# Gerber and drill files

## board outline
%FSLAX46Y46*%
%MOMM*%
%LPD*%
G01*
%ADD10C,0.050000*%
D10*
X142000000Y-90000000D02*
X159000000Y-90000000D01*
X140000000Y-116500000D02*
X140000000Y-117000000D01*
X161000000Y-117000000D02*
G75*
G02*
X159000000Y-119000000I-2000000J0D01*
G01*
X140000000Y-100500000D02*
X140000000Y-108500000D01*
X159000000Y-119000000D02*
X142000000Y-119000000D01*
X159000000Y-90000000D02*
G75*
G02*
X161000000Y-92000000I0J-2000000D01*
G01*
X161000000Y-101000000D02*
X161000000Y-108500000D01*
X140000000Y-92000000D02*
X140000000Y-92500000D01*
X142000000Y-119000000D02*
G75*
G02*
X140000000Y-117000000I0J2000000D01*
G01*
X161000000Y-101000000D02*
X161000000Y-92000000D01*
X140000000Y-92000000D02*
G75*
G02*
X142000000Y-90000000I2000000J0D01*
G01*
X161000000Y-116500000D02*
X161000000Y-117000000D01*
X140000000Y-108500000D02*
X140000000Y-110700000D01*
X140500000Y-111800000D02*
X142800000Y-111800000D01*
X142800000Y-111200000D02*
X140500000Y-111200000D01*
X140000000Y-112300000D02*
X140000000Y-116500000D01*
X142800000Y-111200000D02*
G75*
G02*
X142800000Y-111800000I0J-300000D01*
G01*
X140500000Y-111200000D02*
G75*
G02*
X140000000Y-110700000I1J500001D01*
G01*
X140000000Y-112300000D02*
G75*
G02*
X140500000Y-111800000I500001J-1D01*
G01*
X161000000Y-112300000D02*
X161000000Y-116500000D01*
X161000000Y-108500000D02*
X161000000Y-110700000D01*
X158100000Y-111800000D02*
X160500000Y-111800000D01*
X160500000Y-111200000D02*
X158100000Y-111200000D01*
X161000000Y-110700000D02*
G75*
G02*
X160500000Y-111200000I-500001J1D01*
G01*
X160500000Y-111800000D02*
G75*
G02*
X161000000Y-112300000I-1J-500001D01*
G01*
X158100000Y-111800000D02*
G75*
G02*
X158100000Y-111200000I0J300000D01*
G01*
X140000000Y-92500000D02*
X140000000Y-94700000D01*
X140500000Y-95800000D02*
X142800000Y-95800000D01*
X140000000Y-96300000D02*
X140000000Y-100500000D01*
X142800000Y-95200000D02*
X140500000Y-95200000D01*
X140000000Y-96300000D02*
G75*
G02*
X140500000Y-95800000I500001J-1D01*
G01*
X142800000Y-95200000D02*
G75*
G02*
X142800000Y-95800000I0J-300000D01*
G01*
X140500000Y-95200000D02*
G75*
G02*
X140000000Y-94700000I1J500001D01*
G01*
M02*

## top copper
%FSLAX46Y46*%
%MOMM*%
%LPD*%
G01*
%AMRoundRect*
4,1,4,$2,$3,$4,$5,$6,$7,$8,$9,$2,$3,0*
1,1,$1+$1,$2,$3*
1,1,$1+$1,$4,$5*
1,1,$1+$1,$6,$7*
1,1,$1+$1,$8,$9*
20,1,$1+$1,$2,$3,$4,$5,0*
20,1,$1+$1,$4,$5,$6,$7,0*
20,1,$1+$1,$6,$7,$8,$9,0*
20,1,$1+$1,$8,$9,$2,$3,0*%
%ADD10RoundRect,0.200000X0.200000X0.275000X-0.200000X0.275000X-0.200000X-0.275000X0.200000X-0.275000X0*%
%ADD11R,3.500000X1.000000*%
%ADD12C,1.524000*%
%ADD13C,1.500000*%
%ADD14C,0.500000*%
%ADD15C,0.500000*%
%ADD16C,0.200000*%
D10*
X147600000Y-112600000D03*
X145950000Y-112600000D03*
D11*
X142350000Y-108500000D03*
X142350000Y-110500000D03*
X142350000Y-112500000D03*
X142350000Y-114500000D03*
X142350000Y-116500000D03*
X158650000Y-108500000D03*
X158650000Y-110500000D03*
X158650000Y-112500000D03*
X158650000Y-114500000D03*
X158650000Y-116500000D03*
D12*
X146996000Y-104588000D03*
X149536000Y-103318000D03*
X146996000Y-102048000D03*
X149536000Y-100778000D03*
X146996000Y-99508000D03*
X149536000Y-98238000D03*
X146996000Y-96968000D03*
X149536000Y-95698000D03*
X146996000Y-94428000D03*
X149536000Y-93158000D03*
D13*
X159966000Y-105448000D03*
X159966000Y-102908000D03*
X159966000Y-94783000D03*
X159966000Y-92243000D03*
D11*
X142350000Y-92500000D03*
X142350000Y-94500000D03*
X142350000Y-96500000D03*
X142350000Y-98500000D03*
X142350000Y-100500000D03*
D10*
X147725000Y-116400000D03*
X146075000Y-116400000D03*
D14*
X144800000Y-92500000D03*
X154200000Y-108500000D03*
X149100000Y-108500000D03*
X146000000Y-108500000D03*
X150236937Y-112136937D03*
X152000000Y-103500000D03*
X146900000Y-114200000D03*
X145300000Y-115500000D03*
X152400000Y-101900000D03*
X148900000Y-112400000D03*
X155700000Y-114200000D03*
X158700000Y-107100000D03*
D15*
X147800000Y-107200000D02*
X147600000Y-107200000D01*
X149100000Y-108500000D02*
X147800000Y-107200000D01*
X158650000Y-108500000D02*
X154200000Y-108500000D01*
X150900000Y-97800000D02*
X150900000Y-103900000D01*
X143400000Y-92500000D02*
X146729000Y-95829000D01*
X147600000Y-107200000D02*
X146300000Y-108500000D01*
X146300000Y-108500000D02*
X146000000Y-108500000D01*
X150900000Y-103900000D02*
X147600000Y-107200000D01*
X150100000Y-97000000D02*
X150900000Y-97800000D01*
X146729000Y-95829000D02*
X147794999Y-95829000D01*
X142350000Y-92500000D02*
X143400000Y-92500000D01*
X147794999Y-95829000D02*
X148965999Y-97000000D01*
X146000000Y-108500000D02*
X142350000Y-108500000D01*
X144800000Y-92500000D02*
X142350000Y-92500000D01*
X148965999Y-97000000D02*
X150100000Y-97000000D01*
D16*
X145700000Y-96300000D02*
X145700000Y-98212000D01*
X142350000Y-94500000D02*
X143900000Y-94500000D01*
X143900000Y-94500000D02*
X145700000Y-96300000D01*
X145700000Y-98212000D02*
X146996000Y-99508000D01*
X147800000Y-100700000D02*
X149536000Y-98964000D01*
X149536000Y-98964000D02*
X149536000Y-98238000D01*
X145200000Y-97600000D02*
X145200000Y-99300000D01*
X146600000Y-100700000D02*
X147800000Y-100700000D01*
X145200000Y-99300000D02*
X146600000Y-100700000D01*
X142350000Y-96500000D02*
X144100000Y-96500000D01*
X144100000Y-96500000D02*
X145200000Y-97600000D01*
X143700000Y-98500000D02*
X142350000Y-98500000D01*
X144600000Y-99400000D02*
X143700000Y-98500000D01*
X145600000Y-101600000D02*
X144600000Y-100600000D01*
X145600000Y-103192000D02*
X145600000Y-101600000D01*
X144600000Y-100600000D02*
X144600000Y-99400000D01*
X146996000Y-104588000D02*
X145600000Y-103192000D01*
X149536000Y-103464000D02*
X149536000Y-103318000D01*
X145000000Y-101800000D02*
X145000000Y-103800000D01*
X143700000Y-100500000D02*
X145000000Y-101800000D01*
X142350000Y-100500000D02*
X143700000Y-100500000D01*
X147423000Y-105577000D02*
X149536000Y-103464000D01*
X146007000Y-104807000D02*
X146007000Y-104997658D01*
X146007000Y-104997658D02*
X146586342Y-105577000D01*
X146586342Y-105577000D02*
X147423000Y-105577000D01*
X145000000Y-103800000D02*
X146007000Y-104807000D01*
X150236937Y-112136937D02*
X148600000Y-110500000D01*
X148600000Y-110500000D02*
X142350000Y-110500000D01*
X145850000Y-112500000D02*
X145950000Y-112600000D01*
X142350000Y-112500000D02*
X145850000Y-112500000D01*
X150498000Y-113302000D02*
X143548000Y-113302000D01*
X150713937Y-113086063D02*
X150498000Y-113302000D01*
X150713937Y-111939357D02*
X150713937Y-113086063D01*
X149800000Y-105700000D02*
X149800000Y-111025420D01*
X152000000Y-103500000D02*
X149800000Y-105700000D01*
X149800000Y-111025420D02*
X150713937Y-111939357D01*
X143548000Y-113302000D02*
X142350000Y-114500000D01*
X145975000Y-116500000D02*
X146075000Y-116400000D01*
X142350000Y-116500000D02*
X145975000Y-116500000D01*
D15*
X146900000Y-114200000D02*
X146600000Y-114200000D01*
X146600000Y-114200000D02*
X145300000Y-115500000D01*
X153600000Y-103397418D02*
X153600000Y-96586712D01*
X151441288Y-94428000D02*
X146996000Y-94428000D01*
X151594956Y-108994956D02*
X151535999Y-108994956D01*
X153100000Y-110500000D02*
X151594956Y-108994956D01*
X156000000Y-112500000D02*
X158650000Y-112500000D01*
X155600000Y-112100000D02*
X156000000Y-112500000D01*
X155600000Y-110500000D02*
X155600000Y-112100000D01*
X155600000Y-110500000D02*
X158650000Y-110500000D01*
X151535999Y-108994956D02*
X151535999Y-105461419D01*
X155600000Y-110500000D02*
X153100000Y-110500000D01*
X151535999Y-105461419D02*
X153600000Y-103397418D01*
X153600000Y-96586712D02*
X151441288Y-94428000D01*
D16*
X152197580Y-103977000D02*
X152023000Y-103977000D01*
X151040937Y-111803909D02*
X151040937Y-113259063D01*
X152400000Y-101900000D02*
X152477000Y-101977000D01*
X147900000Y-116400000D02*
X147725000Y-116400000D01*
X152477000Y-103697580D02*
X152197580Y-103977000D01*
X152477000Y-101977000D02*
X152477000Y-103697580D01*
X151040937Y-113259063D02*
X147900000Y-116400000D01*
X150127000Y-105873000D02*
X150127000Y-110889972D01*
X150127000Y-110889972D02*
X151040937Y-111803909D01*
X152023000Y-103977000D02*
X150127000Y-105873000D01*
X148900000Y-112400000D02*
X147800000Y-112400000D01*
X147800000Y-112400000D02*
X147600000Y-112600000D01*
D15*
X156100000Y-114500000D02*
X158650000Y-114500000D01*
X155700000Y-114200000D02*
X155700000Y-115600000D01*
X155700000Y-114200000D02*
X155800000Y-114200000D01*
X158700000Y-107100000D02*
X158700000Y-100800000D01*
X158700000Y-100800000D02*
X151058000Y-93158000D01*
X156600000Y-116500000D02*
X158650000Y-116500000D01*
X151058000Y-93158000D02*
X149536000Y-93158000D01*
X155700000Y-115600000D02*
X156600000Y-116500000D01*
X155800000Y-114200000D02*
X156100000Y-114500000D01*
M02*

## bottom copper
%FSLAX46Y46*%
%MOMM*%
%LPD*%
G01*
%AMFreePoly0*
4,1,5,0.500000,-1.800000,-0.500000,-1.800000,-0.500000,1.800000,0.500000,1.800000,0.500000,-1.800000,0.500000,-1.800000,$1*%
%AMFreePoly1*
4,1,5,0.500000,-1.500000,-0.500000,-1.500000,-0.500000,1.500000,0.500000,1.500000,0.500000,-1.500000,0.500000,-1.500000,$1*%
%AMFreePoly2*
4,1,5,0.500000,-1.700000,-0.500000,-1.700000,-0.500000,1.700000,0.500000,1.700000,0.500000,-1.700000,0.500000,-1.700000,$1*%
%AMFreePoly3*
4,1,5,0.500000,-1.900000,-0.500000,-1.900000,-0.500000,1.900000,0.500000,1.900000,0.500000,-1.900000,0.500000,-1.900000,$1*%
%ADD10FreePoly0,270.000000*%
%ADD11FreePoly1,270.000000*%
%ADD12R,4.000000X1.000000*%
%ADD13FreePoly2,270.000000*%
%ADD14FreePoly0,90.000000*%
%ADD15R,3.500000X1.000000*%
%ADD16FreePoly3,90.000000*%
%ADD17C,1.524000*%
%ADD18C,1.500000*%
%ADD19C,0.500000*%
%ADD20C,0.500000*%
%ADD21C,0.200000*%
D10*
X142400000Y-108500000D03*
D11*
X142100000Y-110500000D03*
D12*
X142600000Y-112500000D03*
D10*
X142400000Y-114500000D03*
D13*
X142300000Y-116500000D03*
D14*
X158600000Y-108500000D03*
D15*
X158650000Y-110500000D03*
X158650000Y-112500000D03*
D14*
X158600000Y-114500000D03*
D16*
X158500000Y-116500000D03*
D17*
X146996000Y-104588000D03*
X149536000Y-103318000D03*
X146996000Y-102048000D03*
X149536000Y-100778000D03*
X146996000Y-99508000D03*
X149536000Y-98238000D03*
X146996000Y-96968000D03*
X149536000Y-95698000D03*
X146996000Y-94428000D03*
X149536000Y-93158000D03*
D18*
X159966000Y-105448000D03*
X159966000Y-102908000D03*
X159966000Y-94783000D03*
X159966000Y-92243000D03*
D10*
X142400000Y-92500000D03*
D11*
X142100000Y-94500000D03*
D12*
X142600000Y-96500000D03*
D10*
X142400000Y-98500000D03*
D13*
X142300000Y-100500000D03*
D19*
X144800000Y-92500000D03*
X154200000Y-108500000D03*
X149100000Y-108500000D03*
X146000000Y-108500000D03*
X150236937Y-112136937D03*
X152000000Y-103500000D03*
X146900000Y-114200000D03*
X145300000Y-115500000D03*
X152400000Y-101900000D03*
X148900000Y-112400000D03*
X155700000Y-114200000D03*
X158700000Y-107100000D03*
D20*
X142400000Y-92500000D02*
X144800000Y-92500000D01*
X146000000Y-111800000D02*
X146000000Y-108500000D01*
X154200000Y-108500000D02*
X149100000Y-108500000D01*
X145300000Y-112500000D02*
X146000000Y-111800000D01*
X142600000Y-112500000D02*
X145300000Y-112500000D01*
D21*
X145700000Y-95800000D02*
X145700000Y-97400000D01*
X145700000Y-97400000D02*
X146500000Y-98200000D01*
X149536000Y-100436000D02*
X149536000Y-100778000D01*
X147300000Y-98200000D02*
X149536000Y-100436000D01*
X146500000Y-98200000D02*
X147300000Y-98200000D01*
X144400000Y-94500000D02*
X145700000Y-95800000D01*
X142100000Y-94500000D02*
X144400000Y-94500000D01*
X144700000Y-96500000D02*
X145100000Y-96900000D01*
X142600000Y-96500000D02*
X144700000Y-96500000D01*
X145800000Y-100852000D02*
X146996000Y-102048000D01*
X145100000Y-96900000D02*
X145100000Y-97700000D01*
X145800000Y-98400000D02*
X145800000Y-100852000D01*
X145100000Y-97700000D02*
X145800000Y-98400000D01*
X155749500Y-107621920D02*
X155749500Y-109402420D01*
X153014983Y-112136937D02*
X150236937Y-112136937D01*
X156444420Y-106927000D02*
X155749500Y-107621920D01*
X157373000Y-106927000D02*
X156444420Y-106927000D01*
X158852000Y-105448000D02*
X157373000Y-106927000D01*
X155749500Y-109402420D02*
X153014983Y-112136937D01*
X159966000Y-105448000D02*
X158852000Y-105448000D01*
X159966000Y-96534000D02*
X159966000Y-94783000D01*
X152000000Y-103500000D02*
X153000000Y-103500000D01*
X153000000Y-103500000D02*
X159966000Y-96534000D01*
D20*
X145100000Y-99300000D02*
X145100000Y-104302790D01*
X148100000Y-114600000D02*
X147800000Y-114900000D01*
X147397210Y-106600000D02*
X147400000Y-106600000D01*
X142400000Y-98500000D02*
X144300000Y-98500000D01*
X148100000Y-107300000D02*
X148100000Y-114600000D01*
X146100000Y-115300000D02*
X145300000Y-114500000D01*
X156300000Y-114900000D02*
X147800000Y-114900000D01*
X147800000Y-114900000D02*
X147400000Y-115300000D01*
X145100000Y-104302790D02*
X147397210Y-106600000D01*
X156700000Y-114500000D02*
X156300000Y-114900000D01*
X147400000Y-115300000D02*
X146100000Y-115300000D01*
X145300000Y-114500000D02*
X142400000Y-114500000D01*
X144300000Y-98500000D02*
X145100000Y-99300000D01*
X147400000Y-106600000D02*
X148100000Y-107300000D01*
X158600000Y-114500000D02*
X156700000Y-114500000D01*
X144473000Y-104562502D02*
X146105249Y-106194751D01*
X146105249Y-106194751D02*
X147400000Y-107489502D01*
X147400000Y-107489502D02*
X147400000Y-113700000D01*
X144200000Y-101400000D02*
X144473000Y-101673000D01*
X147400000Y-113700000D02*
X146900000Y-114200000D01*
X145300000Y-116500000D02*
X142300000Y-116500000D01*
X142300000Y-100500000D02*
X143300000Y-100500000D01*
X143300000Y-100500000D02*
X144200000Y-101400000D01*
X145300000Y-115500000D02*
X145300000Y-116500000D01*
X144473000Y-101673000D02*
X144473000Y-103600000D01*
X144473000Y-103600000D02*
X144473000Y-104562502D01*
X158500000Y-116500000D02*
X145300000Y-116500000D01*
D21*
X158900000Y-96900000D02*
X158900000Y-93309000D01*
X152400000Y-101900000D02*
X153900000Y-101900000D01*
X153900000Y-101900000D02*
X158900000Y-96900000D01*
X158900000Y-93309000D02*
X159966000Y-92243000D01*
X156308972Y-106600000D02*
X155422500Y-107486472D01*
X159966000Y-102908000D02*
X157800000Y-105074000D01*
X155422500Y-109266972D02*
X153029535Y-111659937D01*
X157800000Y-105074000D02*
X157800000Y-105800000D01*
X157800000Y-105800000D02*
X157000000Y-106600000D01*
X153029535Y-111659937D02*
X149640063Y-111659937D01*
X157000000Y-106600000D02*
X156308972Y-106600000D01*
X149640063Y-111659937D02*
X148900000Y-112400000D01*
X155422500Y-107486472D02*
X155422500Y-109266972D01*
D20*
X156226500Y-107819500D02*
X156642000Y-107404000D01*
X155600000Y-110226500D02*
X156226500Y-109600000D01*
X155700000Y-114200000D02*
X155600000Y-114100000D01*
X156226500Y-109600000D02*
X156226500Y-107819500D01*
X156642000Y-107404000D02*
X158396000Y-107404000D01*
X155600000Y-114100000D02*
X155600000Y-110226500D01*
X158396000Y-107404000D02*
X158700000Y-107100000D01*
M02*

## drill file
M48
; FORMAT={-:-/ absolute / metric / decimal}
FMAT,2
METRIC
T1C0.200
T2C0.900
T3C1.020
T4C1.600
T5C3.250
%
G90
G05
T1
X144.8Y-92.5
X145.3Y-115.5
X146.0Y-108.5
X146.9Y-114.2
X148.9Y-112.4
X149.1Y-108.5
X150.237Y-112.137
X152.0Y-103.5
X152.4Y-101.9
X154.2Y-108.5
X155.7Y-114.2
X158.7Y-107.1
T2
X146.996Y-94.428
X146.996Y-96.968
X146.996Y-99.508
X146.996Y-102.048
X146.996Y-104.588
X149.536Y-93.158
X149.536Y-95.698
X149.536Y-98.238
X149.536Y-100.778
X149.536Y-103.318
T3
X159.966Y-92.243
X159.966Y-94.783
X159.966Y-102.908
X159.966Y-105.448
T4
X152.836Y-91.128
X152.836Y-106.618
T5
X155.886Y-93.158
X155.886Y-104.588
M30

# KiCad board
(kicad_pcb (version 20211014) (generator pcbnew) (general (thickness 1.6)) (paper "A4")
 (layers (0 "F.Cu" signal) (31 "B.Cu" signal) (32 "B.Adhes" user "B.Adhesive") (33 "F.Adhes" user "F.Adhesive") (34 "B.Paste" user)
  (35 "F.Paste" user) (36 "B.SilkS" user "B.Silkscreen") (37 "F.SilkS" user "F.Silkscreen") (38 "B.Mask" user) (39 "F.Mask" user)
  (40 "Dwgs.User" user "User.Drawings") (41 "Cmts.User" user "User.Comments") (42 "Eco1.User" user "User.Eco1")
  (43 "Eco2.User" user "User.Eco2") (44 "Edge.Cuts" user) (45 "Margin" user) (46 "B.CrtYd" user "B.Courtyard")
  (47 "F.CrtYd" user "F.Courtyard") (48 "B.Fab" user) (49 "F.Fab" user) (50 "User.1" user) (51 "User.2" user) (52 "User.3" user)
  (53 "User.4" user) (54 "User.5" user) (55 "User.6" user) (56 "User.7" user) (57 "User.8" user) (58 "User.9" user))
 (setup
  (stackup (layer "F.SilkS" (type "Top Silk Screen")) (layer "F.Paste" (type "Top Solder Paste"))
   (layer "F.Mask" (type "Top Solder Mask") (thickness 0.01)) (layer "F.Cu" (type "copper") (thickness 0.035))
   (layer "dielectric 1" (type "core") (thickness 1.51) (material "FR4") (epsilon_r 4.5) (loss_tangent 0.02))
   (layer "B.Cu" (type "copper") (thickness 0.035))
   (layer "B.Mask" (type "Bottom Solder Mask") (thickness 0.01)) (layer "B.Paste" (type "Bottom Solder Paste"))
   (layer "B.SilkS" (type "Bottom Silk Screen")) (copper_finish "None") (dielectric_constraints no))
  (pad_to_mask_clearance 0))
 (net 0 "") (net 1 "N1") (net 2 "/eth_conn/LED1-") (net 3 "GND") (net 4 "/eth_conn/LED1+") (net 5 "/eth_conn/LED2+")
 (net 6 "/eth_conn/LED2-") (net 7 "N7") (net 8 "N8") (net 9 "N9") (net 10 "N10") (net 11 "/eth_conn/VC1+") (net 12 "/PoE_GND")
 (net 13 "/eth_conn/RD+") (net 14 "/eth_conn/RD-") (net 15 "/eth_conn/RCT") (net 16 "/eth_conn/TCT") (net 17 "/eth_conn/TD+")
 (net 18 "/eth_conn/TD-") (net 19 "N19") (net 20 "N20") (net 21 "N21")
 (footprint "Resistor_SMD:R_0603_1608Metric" (layer "F.Cu") (at 146.775 112.6 180)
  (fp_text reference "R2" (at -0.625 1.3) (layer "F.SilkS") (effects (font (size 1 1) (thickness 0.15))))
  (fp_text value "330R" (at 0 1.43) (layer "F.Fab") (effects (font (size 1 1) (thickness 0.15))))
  (pad "1" smd roundrect (at -0.825 0 180) (size 0.8 0.95) (layers "F.Cu" "F.Paste" "F.Mask") (roundrect_rratio 0.25) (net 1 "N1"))
  (pad "2" smd roundrect (at 0.825 0 180) (size 0.8 0.95) (layers "F.Cu" "F.Paste" "F.Mask") (roundrect_rratio 0.25)
   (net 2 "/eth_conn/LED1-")))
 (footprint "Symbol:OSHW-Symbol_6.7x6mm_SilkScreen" (layer "F.Cu") (at 151.9 112)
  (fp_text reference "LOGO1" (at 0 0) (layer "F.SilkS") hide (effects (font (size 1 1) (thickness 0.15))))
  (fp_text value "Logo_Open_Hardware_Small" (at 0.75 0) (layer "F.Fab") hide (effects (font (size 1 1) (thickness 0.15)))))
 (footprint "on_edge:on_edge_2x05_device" (layer "F.Cu") (at 140 112.5 -90)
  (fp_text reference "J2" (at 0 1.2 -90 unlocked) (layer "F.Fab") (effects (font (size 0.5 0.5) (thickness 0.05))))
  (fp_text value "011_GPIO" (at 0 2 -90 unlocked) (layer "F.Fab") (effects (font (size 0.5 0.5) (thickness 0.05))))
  (fp_line (start -4 0) (end -1.8 0) (layer "Edge.Cuts") (width 0.05))
  (fp_line (start -0.7 -0.5) (end -0.7 -2.8) (layer "Edge.Cuts") (width 0.05))
  (fp_line (start -1.3 -2.8) (end -1.3 -0.5) (layer "Edge.Cuts") (width 0.05))
  (fp_line (start -0.2 0) (end 4 0) (layer "Edge.Cuts") (width 0.05))
  (fp_arc (start -1.3 -2.8) (mid -1 -3.1) (end -0.7 -2.8) (layer "Edge.Cuts") (width 0.05))
  (fp_arc (start -1.3 -0.5) (mid -1.446447 -0.146447) (end -1.8 0) (layer "Edge.Cuts") (width 0.05))
  (fp_arc (start -0.2 0) (mid -0.553553 -0.146447) (end -0.7 -0.5) (layer "Edge.Cuts") (width 0.05))
  (pad "1" smd rect (at -4 -2.35 90) (size 1 3.5) (layers "F.Cu" "F.Mask") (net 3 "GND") (zone_connect 0))
  (pad "2" smd rect (at -2 -2.35 270) (size 1 3.5) (layers "F.Cu" "F.Mask") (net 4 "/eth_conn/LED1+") (zone_connect 0))
  (pad "3" smd rect (at 0 -2.35 270) (size 1 3.5) (layers "F.Cu" "F.Mask") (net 2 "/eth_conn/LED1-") (zone_connect 0))
  (pad "4" smd rect (at 2 -2.35 90) (size 1 3.5) (layers "F.Cu" "F.Mask") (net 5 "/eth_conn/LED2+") (zone_connect 0))
  (pad "5" smd rect (at 4 -2.35 90) (size 1 3.5) (layers "F.Cu" "F.Mask") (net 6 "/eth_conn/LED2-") (zone_connect 0))
  (pad "6" smd custom (at -4 -2.4 270) (size 1 3.6) (layers "B.Cu" "B.Mask") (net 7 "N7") (zone_connect 0)
   (options (clearance outline) (anchor rect)) (primitives))
  (pad "7" smd custom (at -2 -2.1 270) (size 1 3) (layers "B.Cu" "B.Mask") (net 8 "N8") (zone_connect 0)
   (options (clearance outline) (anchor rect)) (primitives))
  (pad "8" smd rect (at 0 -2.6 270) (size 1 4) (layers "B.Cu" "B.Mask") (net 3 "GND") (zone_connect 0))
  (pad "9" smd custom (at 2 -2.4 270) (size 1 3.6) (layers "B.Cu" "B.Mask") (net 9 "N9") (zone_connect 0)
   (options (clearance outline) (anchor rect)) (primitives))
  (pad "10" smd custom (at 4 -2.3 270) (size 1 3.4) (layers "B.Cu" "B.Mask") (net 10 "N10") (zone_connect 0)
   (options (clearance outline) (anchor rect)) (primitives)))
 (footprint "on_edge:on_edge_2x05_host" (layer "F.Cu") (at 161 112.5 -90)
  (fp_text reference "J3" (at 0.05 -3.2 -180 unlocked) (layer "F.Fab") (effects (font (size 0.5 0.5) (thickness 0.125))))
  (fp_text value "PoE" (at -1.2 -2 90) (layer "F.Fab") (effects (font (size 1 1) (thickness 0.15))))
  (fp_line (start -0.2 0) (end 4 0) (layer "Edge.Cuts") (width 0.05))
  (fp_line (start -4 0) (end -1.8 0) (layer "Edge.Cuts") (width 0.05))
  (fp_line (start -0.7 2.9) (end -0.7 0.5) (layer "Edge.Cuts") (width 0.05))
  (fp_line (start -1.3 0.5) (end -1.3 2.9) (layer "Edge.Cuts") (width 0.05))
  (fp_arc (start -1.8 0) (mid -1.446447 0.146447) (end -1.3 0.5) (layer "Edge.Cuts") (width 0.05))
  (fp_arc (start -0.7 0.5) (mid -0.553553 0.146447) (end -0.2 0) (layer "Edge.Cuts") (width 0.05))
  (fp_arc (start -0.7 2.9) (mid -1 3.2) (end -1.3 2.9) (layer "Edge.Cuts") (width 0.05))
  (pad "1" smd rect (at -4 2.35 270) (size 1 3.5) (layers "F.Cu" "F.Mask") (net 3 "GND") (zone_connect 0))
  (pad "2" smd rect (at -2 2.35 270) (size 1 3.5) (layers "F.Cu" "F.Mask") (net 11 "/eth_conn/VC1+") (zone_connect 0))
  (pad "3" smd rect (at 0 2.35 270) (size 1 3.5) (layers "F.Cu" "F.Mask") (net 11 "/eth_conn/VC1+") (zone_connect 0))
  (pad "4" smd rect (at 2 2.35 270) (size 1 3.5) (layers "F.Cu" "F.Mask") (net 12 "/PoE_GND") (zone_connect 0))
  (pad "5" smd rect (at 4 2.35 270) (size 1 3.5) (layers "F.Cu" "F.Mask") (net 12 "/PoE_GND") (zone_connect 0))
  (pad "6" smd custom (at -4 2.4 90) (size 1 3.6) (layers "B.Cu" "B.Mask") (zone_connect 0) (options (clearance outline) (anchor rect))
   (primitives))
  (pad "7" smd rect (at -2 2.35 90) (size 1 3.5) (layers "B.Cu" "B.Mask") (zone_connect 0))
  (pad "8" smd rect (at 0 2.35 90) (size 1 3.5) (layers "B.Cu" "B.Mask") (zone_connect 0))
  (pad "9" smd custom (at 2 2.4 90) (size 1 3.6) (layers "B.Cu" "B.Mask") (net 9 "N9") (zone_connect 0)
   (options (clearance outline) (anchor rect)) (primitives))
  (pad "10" smd custom (at 4 2.5 90) (size 1 3.8) (layers "B.Cu" "B.Mask") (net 10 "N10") (zone_connect 0)
   (options (clearance outline) (anchor rect)) (primitives)))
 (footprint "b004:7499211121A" (layer "F.Cu") (at 146.996 94.428 -90)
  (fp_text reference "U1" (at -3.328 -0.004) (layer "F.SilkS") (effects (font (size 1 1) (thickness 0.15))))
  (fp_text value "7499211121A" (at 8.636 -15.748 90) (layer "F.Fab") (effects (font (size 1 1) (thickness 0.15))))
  (pad "" np_thru_hole circle (at 12.19 -5.84 270) (size 1.6 1.6) (drill 1.6) (layers *.Cu *.Mask))
  (pad "" np_thru_hole circle (at 10.16 -8.89 270) (size 3.25 3.25) (drill 3.25) (layers *.Cu *.Mask))
  (pad "" np_thru_hole circle (at -3.3 -5.84 270) (size 1.6 1.6) (drill 1.6) (layers *.Cu *.Mask))
  (pad "" np_thru_hole circle (at -1.27 -8.89 270) (size 3.25 3.25) (drill 3.25) (layers *.Cu *.Mask))
  (pad "1" thru_hole circle (at 10.16 0 270) (size 1.524 1.524) (drill 0.9) (layers *.Cu *.Mask) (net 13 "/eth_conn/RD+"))
  (pad "2" thru_hole circle (at 8.89 -2.54 270) (size 1.524 1.524) (drill 0.9) (layers *.Cu *.Mask) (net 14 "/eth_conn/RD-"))
  (pad "3" thru_hole circle (at 7.62 0 270) (size 1.524 1.524) (drill 0.9) (layers *.Cu *.Mask) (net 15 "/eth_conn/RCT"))
  (pad "4" thru_hole circle (at 6.35 -2.54 270) (size 1.524 1.524) (drill 0.9) (layers *.Cu *.Mask) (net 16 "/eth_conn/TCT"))
  (pad "5" thru_hole circle (at 5.08 0 270) (size 1.524 1.524) (drill 0.9) (layers *.Cu *.Mask) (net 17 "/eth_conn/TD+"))
  (pad "6" thru_hole circle (at 3.81 -2.54 270) (size 1.524 1.524) (drill 0.9) (layers *.Cu *.Mask) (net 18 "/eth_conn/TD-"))
  (pad "7" thru_hole circle (at 2.54 0 270) (size 1.524 1.524) (drill 0.9) (layers *.Cu *.Mask) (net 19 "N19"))
  (pad "8" thru_hole circle (at 1.27 -2.54 270) (size 1.524 1.524) (drill 0.9) (layers *.Cu *.Mask) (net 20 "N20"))
  (pad "9" thru_hole circle (at 0 0 270) (size 1.524 1.524) (drill 0.9) (layers *.Cu *.Mask) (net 11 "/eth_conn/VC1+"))
  (pad "10" thru_hole circle (at -1.27 -2.54 270) (size 1.524 1.524) (drill 0.9) (layers *.Cu *.Mask) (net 12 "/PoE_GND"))
  (pad "11" thru_hole circle (at 11.02 -12.97 270) (size 1.5 1.5) (drill 1.02) (layers *.Cu *.Mask) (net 4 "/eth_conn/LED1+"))
  (pad "12" thru_hole circle (at 8.48 -12.97 270) (size 1.5 1.5) (drill 1.02) (layers *.Cu *.Mask) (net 1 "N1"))
  (pad "13" thru_hole circle (at 0.355 -12.97 270) (size 1.5 1.5) (drill 1.02) (layers *.Cu *.Mask) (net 5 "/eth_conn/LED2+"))
  (pad "14" thru_hole circle (at -2.185 -12.97 270) (size 1.5 1.5) (drill 1.02) (layers *.Cu *.Mask) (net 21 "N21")))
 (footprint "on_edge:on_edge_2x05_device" (layer "F.Cu") (at 140 96.5 -90)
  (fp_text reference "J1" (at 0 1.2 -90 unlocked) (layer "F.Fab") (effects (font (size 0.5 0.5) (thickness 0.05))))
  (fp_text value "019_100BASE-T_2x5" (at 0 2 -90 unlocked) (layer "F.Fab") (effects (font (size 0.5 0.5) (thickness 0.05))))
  (fp_line (start -4 0) (end -1.8 0) (layer "Edge.Cuts") (width 0.05))
  (fp_line (start -0.7 -0.5) (end -0.7 -2.8) (layer "Edge.Cuts") (width 0.05))
  (fp_line (start -0.2 0) (end 4 0) (layer "Edge.Cuts") (width 0.05))
  (fp_line (start -1.3 -2.8) (end -1.3 -0.5) (layer "Edge.Cuts") (width 0.05))
  (fp_arc (start -0.2 0) (mid -0.553553 -0.146447) (end -0.7 -0.5) (layer "Edge.Cuts") (width 0.05))
  (fp_arc (start -1.3 -2.8) (mid -1 -3.1) (end -0.7 -2.8) (layer "Edge.Cuts") (width 0.05))
  (fp_arc (start -1.3 -0.5) (mid -1.446447 -0.146447) (end -1.8 0) (layer "Edge.Cuts") (width 0.05))
  (pad "1" smd rect (at -4 -2.35 90) (size 1 3.5) (layers "F.Cu" "F.Mask") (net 3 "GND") (zone_connect 0))
  (pad "2" smd rect (at -2 -2.35 270) (size 1 3.5) (layers "F.Cu" "F.Mask") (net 17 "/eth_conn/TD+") (zone_connect 0))
  (pad "3" smd rect (at 0 -2.35 270) (size 1 3.5) (layers "F.Cu" "F.Mask") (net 18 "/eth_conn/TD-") (zone_connect 0))
  (pad "4" smd rect (at 2 -2.35 90) (size 1 3.5) (layers "F.Cu" "F.Mask") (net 13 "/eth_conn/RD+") (zone_connect 0))
  (pad "5" smd rect (at 4 -2.35 90) (size 1 3.5) (layers "F.Cu" "F.Mask") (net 14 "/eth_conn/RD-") (zone_connect 0))
  (pad "6" smd custom (at -4 -2.4 270) (size 1 3.6) (layers "B.Cu" "B.Mask") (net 3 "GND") (zone_connect 0)
   (options (clearance outline) (anchor rect)) (primitives))
  (pad "7" smd custom (at -2 -2.1 270) (size 1 3) (layers "B.Cu" "B.Mask") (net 16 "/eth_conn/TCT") (zone_connect 0)
   (options (clearance outline) (anchor rect)) (primitives))
  (pad "8" smd rect (at 0 -2.6 270) (size 1 4) (layers "B.Cu" "B.Mask") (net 15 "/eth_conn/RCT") (zone_connect 0))
  (pad "9" smd custom (at 2 -2.4 270) (size 1 3.6) (layers "B.Cu" "B.Mask") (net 9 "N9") (zone_connect 0)
   (options (clearance outline) (anchor rect)) (primitives))
  (pad "10" smd custom (at 4 -2.3 270) (size 1 3.4) (layers "B.Cu" "B.Mask") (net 10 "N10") (zone_connect 0)
   (options (clearance outline) (anchor rect)) (primitives)))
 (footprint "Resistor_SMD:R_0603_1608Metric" (layer "F.Cu") (at 146.9 116.4 180)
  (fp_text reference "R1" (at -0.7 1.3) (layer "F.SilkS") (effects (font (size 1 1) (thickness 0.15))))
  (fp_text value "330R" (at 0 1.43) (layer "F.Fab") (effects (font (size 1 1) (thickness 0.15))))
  (pad "1" smd roundrect (at -0.825 0 180) (size 0.8 0.95) (layers "F.Cu" "F.Paste" "F.Mask") (roundrect_rratio 0.25) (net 21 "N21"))
  (pad "2" smd roundrect (at 0.825 0 180) (size 0.8 0.95) (layers "F.Cu" "F.Paste" "F.Mask") (roundrect_rratio 0.25)
   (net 6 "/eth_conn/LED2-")))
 (gr_line (start 142 90) (end 159 90) (layer "Edge.Cuts") (width 0.05))
 (gr_line (start 140 116.5) (end 140 117) (layer "Edge.Cuts") (width 0.05))
 (gr_arc (start 161 117) (mid 160.414214 118.414214) (end 159 119) (layer "Edge.Cuts") (width 0.05))
 (gr_line (start 140 100.5) (end 140 108.5) (layer "Edge.Cuts") (width 0.05))
 (gr_line (start 159 119) (end 142 119) (layer "Edge.Cuts") (width 0.05))
 (gr_arc (start 159 90) (mid 160.414214 90.585786) (end 161 92) (layer "Edge.Cuts") (width 0.05))
 (gr_line (start 161 101) (end 161 108.5) (layer "Edge.Cuts") (width 0.05))
 (gr_line (start 140 92) (end 140 92.5) (layer "Edge.Cuts") (width 0.05))
 (gr_arc (start 142 119) (mid 140.585786 118.414214) (end 140 117) (layer "Edge.Cuts") (width 0.05))
 (gr_line (start 161 101) (end 161 92) (layer "Edge.Cuts") (width 0.05))
 (gr_arc (start 140 92) (mid 140.585786 90.585786) (end 142 90) (layer "Edge.Cuts") (width 0.05))
 (gr_line (start 161 116.5) (end 161 117) (layer "Edge.Cuts") (width 0.05))
 (segment (start 147.8 107.2) (end 147.6 107.2) (width 0.5) (layer "F.Cu") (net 3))
 (segment (start 149.1 108.5) (end 147.8 107.2) (width 0.5) (layer "F.Cu") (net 3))
 (segment (start 158.65 108.5) (end 154.2 108.5) (width 0.5) (layer "F.Cu") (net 3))
 (segment (start 150.9 97.8) (end 150.9 103.9) (width 0.5) (layer "F.Cu") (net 3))
 (segment (start 143.4 92.5) (end 146.729 95.829) (width 0.5) (layer "F.Cu") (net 3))
 (segment (start 147.6 107.2) (end 146.3 108.5) (width 0.5) (layer "F.Cu") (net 3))
 (segment (start 146.3 108.5) (end 146 108.5) (width 0.5) (layer "F.Cu") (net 3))
 (segment (start 150.9 103.9) (end 147.6 107.2) (width 0.5) (layer "F.Cu") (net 3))
 (segment (start 150.1 97) (end 150.9 97.8) (width 0.5) (layer "F.Cu") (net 3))
 (segment (start 146.729 95.829) (end 147.794999 95.829) (width 0.5) (layer "F.Cu") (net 3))
 (segment (start 142.35 92.5) (end 143.4 92.5) (width 0.5) (layer "F.Cu") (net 3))
 (segment (start 147.794999 95.829) (end 148.965999 97) (width 0.5) (layer "F.Cu") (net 3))
 (segment (start 146 108.5) (end 142.35 108.5) (width 0.5) (layer "F.Cu") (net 3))
 (segment (start 144.8 92.5) (end 142.35 92.5) (width 0.5) (layer "F.Cu") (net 3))
 (segment (start 148.965999 97) (end 150.1 97) (width 0.5) (layer "F.Cu") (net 3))
 (via (at 144.8 92.5) (size 0.5) (drill 0.2) (layers "F.Cu" "B.Cu") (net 3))
 (via (at 154.2 108.5) (size 0.5) (drill 0.2) (layers "F.Cu" "B.Cu") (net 3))
 (via (at 149.1 108.5) (size 0.5) (drill 0.2) (layers "F.Cu" "B.Cu") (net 3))
 (via (at 146 108.5) (size 0.5) (drill 0.2) (layers "F.Cu" "B.Cu") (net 3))
 (segment (start 142.4 92.5) (end 144.8 92.5) (width 0.5) (layer "B.Cu") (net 3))
 (segment (start 146 111.8) (end 146 108.5) (width 0.5) (layer "B.Cu") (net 3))
 (segment (start 154.2 108.5) (end 149.1 108.5) (width 0.5) (layer "B.Cu") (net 3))
 (segment (start 145.3 112.5) (end 146 111.8) (width 0.5) (layer "B.Cu") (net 3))
 (segment (start 142.6 112.5) (end 145.3 112.5) (width 0.5) (layer "B.Cu") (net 3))
 (segment (start 145.7 96.3) (end 145.7 98.212) (width 0.2) (layer "F.Cu") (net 17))
 (segment (start 142.35 94.5) (end 143.9 94.5) (width 0.2) (layer "F.Cu") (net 17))
 (segment (start 143.9 94.5) (end 145.7 96.3) (width 0.2) (layer "F.Cu") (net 17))
 (segment (start 145.7 98.212) (end 146.996 99.508) (width 0.2) (layer "F.Cu") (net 17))
 (segment (start 147.8 100.7) (end 149.536 98.964) (width 0.2) (layer "F.Cu") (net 18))
 (segment (start 149.536 98.964) (end 149.536 98.238) (width 0.2) (layer "F.Cu") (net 18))
 (segment (start 145.2 97.6) (end 145.2 99.3) (width 0.2) (layer "F.Cu") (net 18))
 (segment (start 146.6 100.7) (end 147.8 100.7) (width 0.2) (layer "F.Cu") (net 18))
 (segment (start 145.2 99.3) (end 146.6 100.7) (width 0.2) (layer "F.Cu") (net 18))
 (segment (start 142.35 96.5) (end 144.1 96.5) (width 0.2) (layer "F.Cu") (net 18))
 (segment (start 144.1 96.5) (end 145.2 97.6) (width 0.2) (layer "F.Cu") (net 18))
 (segment (start 143.7 98.5) (end 142.35 98.5) (width 0.2) (layer "F.Cu") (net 13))
 (segment (start 144.6 99.4) (end 143.7 98.5) (width 0.2) (layer "F.Cu") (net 13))
 (segment (start 145.6 101.6) (end 144.6 100.6) (width 0.2) (layer "F.Cu") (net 13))
 (segment (start 145.6 103.192) (end 145.6 101.6) (width 0.2) (layer "F.Cu") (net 13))
 (segment (start 144.6 100.6) (end 144.6 99.4) (width 0.2) (layer "F.Cu") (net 13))
 (segment (start 146.996 104.588) (end 145.6 103.192) (width 0.2) (layer "F.Cu") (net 13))
 (segment (start 149.536 103.464) (end 149.536 103.318) (width 0.2) (layer "F.Cu") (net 14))
 (segment (start 145 101.8) (end 145 103.8) (width 0.2) (layer "F.Cu") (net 14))
 (segment (start 143.7 100.5) (end 145 101.8) (width 0.2) (layer "F.Cu") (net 14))
 (segment (start 142.35 100.5) (end 143.7 100.5) (width 0.2) (layer "F.Cu") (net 14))
 (segment (start 147.423 105.577) (end 149.536 103.464) (width 0.2) (layer "F.Cu") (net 14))
 (segment (start 146.007 104.807) (end 146.007 104.997658) (width 0.2) (layer "F.Cu") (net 14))
 (segment (start 146.007 104.997658) (end 146.586342 105.577) (width 0.2) (layer "F.Cu") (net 14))
 (segment (start 146.586342 105.577) (end 147.423 105.577) (width 0.2) (layer "F.Cu") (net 14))
 (segment (start 145 103.8) (end 146.007 104.807) (width 0.2) (layer "F.Cu") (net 14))
 (segment (start 145.7 95.8) (end 145.7 97.4) (width 0.2) (layer "B.Cu") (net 16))
 (segment (start 145.7 97.4) (end 146.5 98.2) (width 0.2) (layer "B.Cu") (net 16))
 (segment (start 149.536 100.436) (end 149.536 100.778) (width 0.2) (layer "B.Cu") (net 16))
 (segment (start 147.3 98.2) (end 149.536 100.436) (width 0.2) (layer "B.Cu") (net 16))
 (segment (start 146.5 98.2) (end 147.3 98.2) (width 0.2) (layer "B.Cu") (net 16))
 (segment (start 144.4 94.5) (end 145.7 95.8) (width 0.2) (layer "B.Cu") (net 16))
 (segment (start 142.1 94.5) (end 144.4 94.5) (width 0.2) (layer "B.Cu") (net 16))
 (segment (start 144.7 96.5) (end 145.1 96.9) (width 0.2) (layer "B.Cu") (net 15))
 (segment (start 142.6 96.5) (end 144.7 96.5) (width 0.2) (layer "B.Cu") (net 15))
 (segment (start 145.8 100.852) (end 146.996 102.048) (width 0.2) (layer "B.Cu") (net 15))
 (segment (start 145.1 96.9) (end 145.1 97.7) (width 0.2) (layer "B.Cu") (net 15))
 (segment (start 145.8 98.4) (end 145.8 100.852) (width 0.2) (layer "B.Cu") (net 15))
 (segment (start 145.1 97.7) (end 145.8 98.4) (width 0.2) (layer "B.Cu") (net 15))
 (segment (start 150.236937 112.136937) (end 148.6 110.5) (width 0.2) (layer "F.Cu") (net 4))
 (segment (start 148.6 110.5) (end 142.35 110.5) (width 0.2) (layer "F.Cu") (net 4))
 (via (at 150.236937 112.136937) (size 0.5) (drill 0.2) (layers "F.Cu" "B.Cu") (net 4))
 (segment (start 155.7495 107.62192) (end 155.7495 109.40242) (width 0.2) (layer "B.Cu") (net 4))
 (segment (start 153.014983 112.136937) (end 150.236937 112.136937) (width 0.2) (layer "B.Cu") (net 4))
 (segment (start 156.44442 106.927) (end 155.7495 107.62192) (width 0.2) (layer "B.Cu") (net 4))
 (segment (start 157.373 106.927) (end 156.44442 106.927) (width 0.2) (layer "B.Cu") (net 4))
 (segment (start 158.852 105.448) (end 157.373 106.927) (width 0.2) (layer "B.Cu") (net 4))
 (segment (start 155.7495 109.40242) (end 153.014983 112.136937) (width 0.2) (layer "B.Cu") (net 4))
 (segment (start 159.966 105.448) (end 158.852 105.448) (width 0.2) (layer "B.Cu") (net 4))
 (segment (start 145.85 112.5) (end 145.95 112.6) (width 0.2) (layer "F.Cu") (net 2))
 (segment (start 142.35 112.5) (end 145.85 112.5) (width 0.2) (layer "F.Cu") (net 2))
 (segment (start 150.498 113.302) (end 143.548 113.302) (width 0.2) (layer "F.Cu") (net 5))
 (segment (start 150.713937 113.086063) (end 150.498 113.302) (width 0.2) (layer "F.Cu") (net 5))
 (segment (start 150.713937 111.939357) (end 150.713937 113.086063) (width 0.2) (layer "F.Cu") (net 5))
 (segment (start 149.8 105.7) (end 149.8 111.02542) (width 0.2) (layer "F.Cu") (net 5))
 (segment (start 152 103.5) (end 149.8 105.7) (width 0.2) (layer "F.Cu") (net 5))
 (segment (start 149.8 111.02542) (end 150.713937 111.939357) (width 0.2) (layer "F.Cu") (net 5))
 (segment (start 143.548 113.302) (end 142.35 114.5) (width 0.2) (layer "F.Cu") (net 5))
 (via (at 152 103.5) (size 0.5) (drill 0.2) (layers "F.Cu" "B.Cu") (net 5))
 (segment (start 159.966 96.534) (end 159.966 94.783) (width 0.2) (layer "B.Cu") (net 5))
 (segment (start 152 103.5) (end 153 103.5) (width 0.2) (layer "B.Cu") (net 5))
 (segment (start 153 103.5) (end 159.966 96.534) (width 0.2) (layer "B.Cu") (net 5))
 (segment (start 145.975 116.5) (end 146.075 116.4) (width 0.2) (layer "F.Cu") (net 6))
 (segment (start 142.35 116.5) (end 145.975 116.5) (width 0.2) (layer "F.Cu") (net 6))
 (segment (start 145.1 99.3) (end 145.1 104.30279) (width 0.5) (layer "B.Cu") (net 9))
 (segment (start 148.1 114.6) (end 147.8 114.9) (width 0.5) (layer "B.Cu") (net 9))
 (segment (start 147.39721 106.6) (end 147.4 106.6) (width 0.5) (layer "B.Cu") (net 9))
 (segment (start 142.4 98.5) (end 144.3 98.5) (width 0.5) (layer "B.Cu") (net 9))
 (segment (start 148.1 107.3) (end 148.1 114.6) (width 0.5) (layer "B.Cu") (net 9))
 (segment (start 146.1 115.3) (end 145.3 114.5) (width 0.5) (layer "B.Cu") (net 9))
 (segment (start 156.3 114.9) (end 147.8 114.9) (width 0.5) (layer "B.Cu") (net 9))
 (segment (start 147.8 114.9) (end 147.4 115.3) (width 0.5) (layer "B.Cu") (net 9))
 (segment (start 145.1 104.30279) (end 147.39721 106.6) (width 0.5) (layer "B.Cu") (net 9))
 (segment (start 156.7 114.5) (end 156.3 114.9) (width 0.5) (layer "B.Cu") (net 9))
 (segment (start 147.4 115.3) (end 146.1 115.3) (width 0.5) (layer "B.Cu") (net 9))
 (segment (start 145.3 114.5) (end 142.4 114.5) (width 0.5) (layer "B.Cu") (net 9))
 (segment (start 144.3 98.5) (end 145.1 99.3) (width 0.5) (layer "B.Cu") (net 9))
 (segment (start 147.4 106.6) (end 148.1 107.3) (width 0.5) (layer "B.Cu") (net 9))
 (segment (start 158.6 114.5) (end 156.7 114.5) (width 0.5) (layer "B.Cu") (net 9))
 (segment (start 146.9 114.2) (end 146.6 114.2) (width 0.5) (layer "F.Cu") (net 10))
 (segment (start 146.6 114.2) (end 145.3 115.5) (width 0.5) (layer "F.Cu") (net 10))
 (via (at 146.9 114.2) (size 0.5) (drill 0.2) (layers "F.Cu" "B.Cu") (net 10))
 (via (at 145.3 115.5) (size 0.5) (drill 0.2) (layers "F.Cu" "B.Cu") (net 10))
 (segment (start 144.473 104.562502) (end 146.105249 106.194751) (width 0.5) (layer "B.Cu") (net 10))
 (segment (start 146.105249 106.194751) (end 147.4 107.489502) (width 0.5) (layer "B.Cu") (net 10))
 (segment (start 147.4 107.489502) (end 147.4 113.7) (width 0.5) (layer "B.Cu") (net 10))
 (segment (start 144.2 101.4) (end 144.473 101.673) (width 0.5) (layer "B.Cu") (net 10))
 (segment (start 147.4 113.7) (end 146.9 114.2) (width 0.5) (layer "B.Cu") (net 10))
 (segment (start 145.3 116.5) (end 142.3 116.5) (width 0.5) (layer "B.Cu") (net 10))
 (segment (start 142.3 100.5) (end 143.3 100.5) (width 0.5) (layer "B.Cu") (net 10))
 (segment (start 143.3 100.5) (end 144.2 101.4) (width 0.5) (layer "B.Cu") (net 10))
 (segment (start 145.3 115.5) (end 145.3 116.5) (width 0.5) (layer "B.Cu") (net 10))
 (segment (start 144.473 101.673) (end 144.473 103.6) (width 0.5) (layer "B.Cu") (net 10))
 (segment (start 144.473 103.6) (end 144.473 104.562502) (width 0.5) (layer "B.Cu") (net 10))
 (segment (start 158.5 116.5) (end 145.3 116.5) (width 0.5) (layer "B.Cu") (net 10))
 (segment (start 153.6 103.397418) (end 153.6 96.586712) (width 0.5) (layer "F.Cu") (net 11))
 (segment (start 151.441288 94.428) (end 146.996 94.428) (width 0.5) (layer "F.Cu") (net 11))
 (segment (start 151.594956 108.994956) (end 151.535999 108.994956) (width 0.5) (layer "F.Cu") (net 11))
 (segment (start 153.1 110.5) (end 151.594956 108.994956) (width 0.5) (layer "F.Cu") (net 11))
 (segment (start 156 112.5) (end 158.65 112.5) (width 0.5) (layer "F.Cu") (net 11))
 (segment (start 155.6 112.1) (end 156 112.5) (width 0.5) (layer "F.Cu") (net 11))
 (segment (start 155.6 110.5) (end 155.6 112.1) (width 0.5) (layer "F.Cu") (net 11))
 (segment (start 155.6 110.5) (end 158.65 110.5) (width 0.5) (layer "F.Cu") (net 11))
 (segment (start 151.535999 108.994956) (end 151.535999 105.461419) (width 0.5) (layer "F.Cu") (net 11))
 (segment (start 155.6 110.5) (end 153.1 110.5) (width 0.5) (layer "F.Cu") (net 11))
 (segment (start 151.535999 105.461419) (end 153.6 103.397418) (width 0.5) (layer "F.Cu") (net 11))
 (segment (start 153.6 96.586712) (end 151.441288 94.428) (width 0.5) (layer "F.Cu") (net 11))
 (segment (start 152.19758 103.977) (end 152.023 103.977) (width 0.2) (layer "F.Cu") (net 21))
 (segment (start 151.040937 111.803909) (end 151.040937 113.259063) (width 0.2) (layer "F.Cu") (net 21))
 (segment (start 152.4 101.9) (end 152.477 101.977) (width 0.2) (layer "F.Cu") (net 21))
 (segment (start 147.9 116.4) (end 147.725 116.4) (width 0.2) (layer "F.Cu") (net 21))
 (segment (start 152.477 103.69758) (end 152.19758 103.977) (width 0.2) (layer "F.Cu") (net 21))
 (segment (start 152.477 101.977) (end 152.477 103.69758) (width 0.2) (layer "F.Cu") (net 21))
 (segment (start 151.040937 113.259063) (end 147.9 116.4) (width 0.2) (layer "F.Cu") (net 21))
 (segment (start 150.127 105.873) (end 150.127 110.889972) (width 0.2) (layer "F.Cu") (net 21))
 (segment (start 150.127 110.889972) (end 151.040937 111.803909) (width 0.2) (layer "F.Cu") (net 21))
 (segment (start 152.023 103.977) (end 150.127 105.873) (width 0.2) (layer "F.Cu") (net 21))
 (via (at 152.4 101.9) (size 0.5) (drill 0.2) (layers "F.Cu" "B.Cu") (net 21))
 (segment (start 158.9 96.9) (end 158.9 93.309) (width 0.2) (layer "B.Cu") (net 21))
 (segment (start 152.4 101.9) (end 153.9 101.9) (width 0.2) (layer "B.Cu") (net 21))
 (segment (start 153.9 101.9) (end 158.9 96.9) (width 0.2) (layer "B.Cu") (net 21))
 (segment (start 158.9 93.309) (end 159.966 92.243) (width 0.2) (layer "B.Cu") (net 21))
 (segment (start 148.9 112.4) (end 147.8 112.4) (width 0.2) (layer "F.Cu") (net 1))
 (segment (start 147.8 112.4) (end 147.6 112.6) (width 0.2) (layer "F.Cu") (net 1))
 (via (at 148.9 112.4) (size 0.5) (drill 0.2) (layers "F.Cu" "B.Cu") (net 1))
 (segment (start 156.308972 106.6) (end 155.4225 107.486472) (width 0.2) (layer "B.Cu") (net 1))
 (segment (start 159.966 102.908) (end 157.8 105.074) (width 0.2) (layer "B.Cu") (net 1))
 (segment (start 155.4225 109.266972) (end 153.029535 111.659937) (width 0.2) (layer "B.Cu") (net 1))
 (segment (start 157.8 105.074) (end 157.8 105.8) (width 0.2) (layer "B.Cu") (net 1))
 (segment (start 157.8 105.8) (end 157 106.6) (width 0.2) (layer "B.Cu") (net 1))
 (segment (start 153.029535 111.659937) (end 149.640063 111.659937) (width 0.2) (layer "B.Cu") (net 1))
 (segment (start 157 106.6) (end 156.308972 106.6) (width 0.2) (layer "B.Cu") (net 1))
 (segment (start 149.640063 111.659937) (end 148.9 112.4) (width 0.2) (layer "B.Cu") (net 1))
 (segment (start 155.4225 107.486472) (end 155.4225 109.266972) (width 0.2) (layer "B.Cu") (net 1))
 (segment (start 156.1 114.5) (end 158.65 114.5) (width 0.5) (layer "F.Cu") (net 12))
 (segment (start 155.7 114.2) (end 155.7 115.6) (width 0.5) (layer "F.Cu") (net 12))
 (segment (start 155.7 114.2) (end 155.8 114.2) (width 0.5) (layer "F.Cu") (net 12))
 (segment (start 158.7 107.1) (end 158.7 100.8) (width 0.5) (layer "F.Cu") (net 12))
 (segment (start 158.7 100.8) (end 151.058 93.158) (width 0.5) (layer "F.Cu") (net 12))
 (segment (start 156.6 116.5) (end 158.65 116.5) (width 0.5) (layer "F.Cu") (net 12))
 (segment (start 151.058 93.158) (end 149.536 93.158) (width 0.5) (layer "F.Cu") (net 12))
 (segment (start 155.7 115.6) (end 156.6 116.5) (width 0.5) (layer "F.Cu") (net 12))
 (segment (start 155.8 114.2) (end 156.1 114.5) (width 0.5) (layer "F.Cu") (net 12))
 (via (at 155.7 114.2) (size 0.5) (drill 0.2) (layers "F.Cu" "B.Cu") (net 12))
 (via (at 158.7 107.1) (size 0.5) (drill 0.2) (layers "F.Cu" "B.Cu") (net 12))
 (segment (start 156.2265 107.8195) (end 156.642 107.404) (width 0.5) (layer "B.Cu") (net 12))
 (segment (start 155.6 110.2265) (end 156.2265 109.6) (width 0.5) (layer "B.Cu") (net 12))
 (segment (start 155.7 114.2) (end 155.6 114.1) (width 0.5) (layer "B.Cu") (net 12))
 (segment (start 156.2265 109.6) (end 156.2265 107.8195) (width 0.5) (layer "B.Cu") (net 12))
 (segment (start 156.642 107.404) (end 158.396 107.404) (width 0.5) (layer "B.Cu") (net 12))
 (segment (start 155.6 114.1) (end 155.6 110.2265) (width 0.5) (layer "B.Cu") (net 12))
 (segment (start 158.396 107.404) (end 158.7 107.1) (width 0.5) (layer "B.Cu") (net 12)))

